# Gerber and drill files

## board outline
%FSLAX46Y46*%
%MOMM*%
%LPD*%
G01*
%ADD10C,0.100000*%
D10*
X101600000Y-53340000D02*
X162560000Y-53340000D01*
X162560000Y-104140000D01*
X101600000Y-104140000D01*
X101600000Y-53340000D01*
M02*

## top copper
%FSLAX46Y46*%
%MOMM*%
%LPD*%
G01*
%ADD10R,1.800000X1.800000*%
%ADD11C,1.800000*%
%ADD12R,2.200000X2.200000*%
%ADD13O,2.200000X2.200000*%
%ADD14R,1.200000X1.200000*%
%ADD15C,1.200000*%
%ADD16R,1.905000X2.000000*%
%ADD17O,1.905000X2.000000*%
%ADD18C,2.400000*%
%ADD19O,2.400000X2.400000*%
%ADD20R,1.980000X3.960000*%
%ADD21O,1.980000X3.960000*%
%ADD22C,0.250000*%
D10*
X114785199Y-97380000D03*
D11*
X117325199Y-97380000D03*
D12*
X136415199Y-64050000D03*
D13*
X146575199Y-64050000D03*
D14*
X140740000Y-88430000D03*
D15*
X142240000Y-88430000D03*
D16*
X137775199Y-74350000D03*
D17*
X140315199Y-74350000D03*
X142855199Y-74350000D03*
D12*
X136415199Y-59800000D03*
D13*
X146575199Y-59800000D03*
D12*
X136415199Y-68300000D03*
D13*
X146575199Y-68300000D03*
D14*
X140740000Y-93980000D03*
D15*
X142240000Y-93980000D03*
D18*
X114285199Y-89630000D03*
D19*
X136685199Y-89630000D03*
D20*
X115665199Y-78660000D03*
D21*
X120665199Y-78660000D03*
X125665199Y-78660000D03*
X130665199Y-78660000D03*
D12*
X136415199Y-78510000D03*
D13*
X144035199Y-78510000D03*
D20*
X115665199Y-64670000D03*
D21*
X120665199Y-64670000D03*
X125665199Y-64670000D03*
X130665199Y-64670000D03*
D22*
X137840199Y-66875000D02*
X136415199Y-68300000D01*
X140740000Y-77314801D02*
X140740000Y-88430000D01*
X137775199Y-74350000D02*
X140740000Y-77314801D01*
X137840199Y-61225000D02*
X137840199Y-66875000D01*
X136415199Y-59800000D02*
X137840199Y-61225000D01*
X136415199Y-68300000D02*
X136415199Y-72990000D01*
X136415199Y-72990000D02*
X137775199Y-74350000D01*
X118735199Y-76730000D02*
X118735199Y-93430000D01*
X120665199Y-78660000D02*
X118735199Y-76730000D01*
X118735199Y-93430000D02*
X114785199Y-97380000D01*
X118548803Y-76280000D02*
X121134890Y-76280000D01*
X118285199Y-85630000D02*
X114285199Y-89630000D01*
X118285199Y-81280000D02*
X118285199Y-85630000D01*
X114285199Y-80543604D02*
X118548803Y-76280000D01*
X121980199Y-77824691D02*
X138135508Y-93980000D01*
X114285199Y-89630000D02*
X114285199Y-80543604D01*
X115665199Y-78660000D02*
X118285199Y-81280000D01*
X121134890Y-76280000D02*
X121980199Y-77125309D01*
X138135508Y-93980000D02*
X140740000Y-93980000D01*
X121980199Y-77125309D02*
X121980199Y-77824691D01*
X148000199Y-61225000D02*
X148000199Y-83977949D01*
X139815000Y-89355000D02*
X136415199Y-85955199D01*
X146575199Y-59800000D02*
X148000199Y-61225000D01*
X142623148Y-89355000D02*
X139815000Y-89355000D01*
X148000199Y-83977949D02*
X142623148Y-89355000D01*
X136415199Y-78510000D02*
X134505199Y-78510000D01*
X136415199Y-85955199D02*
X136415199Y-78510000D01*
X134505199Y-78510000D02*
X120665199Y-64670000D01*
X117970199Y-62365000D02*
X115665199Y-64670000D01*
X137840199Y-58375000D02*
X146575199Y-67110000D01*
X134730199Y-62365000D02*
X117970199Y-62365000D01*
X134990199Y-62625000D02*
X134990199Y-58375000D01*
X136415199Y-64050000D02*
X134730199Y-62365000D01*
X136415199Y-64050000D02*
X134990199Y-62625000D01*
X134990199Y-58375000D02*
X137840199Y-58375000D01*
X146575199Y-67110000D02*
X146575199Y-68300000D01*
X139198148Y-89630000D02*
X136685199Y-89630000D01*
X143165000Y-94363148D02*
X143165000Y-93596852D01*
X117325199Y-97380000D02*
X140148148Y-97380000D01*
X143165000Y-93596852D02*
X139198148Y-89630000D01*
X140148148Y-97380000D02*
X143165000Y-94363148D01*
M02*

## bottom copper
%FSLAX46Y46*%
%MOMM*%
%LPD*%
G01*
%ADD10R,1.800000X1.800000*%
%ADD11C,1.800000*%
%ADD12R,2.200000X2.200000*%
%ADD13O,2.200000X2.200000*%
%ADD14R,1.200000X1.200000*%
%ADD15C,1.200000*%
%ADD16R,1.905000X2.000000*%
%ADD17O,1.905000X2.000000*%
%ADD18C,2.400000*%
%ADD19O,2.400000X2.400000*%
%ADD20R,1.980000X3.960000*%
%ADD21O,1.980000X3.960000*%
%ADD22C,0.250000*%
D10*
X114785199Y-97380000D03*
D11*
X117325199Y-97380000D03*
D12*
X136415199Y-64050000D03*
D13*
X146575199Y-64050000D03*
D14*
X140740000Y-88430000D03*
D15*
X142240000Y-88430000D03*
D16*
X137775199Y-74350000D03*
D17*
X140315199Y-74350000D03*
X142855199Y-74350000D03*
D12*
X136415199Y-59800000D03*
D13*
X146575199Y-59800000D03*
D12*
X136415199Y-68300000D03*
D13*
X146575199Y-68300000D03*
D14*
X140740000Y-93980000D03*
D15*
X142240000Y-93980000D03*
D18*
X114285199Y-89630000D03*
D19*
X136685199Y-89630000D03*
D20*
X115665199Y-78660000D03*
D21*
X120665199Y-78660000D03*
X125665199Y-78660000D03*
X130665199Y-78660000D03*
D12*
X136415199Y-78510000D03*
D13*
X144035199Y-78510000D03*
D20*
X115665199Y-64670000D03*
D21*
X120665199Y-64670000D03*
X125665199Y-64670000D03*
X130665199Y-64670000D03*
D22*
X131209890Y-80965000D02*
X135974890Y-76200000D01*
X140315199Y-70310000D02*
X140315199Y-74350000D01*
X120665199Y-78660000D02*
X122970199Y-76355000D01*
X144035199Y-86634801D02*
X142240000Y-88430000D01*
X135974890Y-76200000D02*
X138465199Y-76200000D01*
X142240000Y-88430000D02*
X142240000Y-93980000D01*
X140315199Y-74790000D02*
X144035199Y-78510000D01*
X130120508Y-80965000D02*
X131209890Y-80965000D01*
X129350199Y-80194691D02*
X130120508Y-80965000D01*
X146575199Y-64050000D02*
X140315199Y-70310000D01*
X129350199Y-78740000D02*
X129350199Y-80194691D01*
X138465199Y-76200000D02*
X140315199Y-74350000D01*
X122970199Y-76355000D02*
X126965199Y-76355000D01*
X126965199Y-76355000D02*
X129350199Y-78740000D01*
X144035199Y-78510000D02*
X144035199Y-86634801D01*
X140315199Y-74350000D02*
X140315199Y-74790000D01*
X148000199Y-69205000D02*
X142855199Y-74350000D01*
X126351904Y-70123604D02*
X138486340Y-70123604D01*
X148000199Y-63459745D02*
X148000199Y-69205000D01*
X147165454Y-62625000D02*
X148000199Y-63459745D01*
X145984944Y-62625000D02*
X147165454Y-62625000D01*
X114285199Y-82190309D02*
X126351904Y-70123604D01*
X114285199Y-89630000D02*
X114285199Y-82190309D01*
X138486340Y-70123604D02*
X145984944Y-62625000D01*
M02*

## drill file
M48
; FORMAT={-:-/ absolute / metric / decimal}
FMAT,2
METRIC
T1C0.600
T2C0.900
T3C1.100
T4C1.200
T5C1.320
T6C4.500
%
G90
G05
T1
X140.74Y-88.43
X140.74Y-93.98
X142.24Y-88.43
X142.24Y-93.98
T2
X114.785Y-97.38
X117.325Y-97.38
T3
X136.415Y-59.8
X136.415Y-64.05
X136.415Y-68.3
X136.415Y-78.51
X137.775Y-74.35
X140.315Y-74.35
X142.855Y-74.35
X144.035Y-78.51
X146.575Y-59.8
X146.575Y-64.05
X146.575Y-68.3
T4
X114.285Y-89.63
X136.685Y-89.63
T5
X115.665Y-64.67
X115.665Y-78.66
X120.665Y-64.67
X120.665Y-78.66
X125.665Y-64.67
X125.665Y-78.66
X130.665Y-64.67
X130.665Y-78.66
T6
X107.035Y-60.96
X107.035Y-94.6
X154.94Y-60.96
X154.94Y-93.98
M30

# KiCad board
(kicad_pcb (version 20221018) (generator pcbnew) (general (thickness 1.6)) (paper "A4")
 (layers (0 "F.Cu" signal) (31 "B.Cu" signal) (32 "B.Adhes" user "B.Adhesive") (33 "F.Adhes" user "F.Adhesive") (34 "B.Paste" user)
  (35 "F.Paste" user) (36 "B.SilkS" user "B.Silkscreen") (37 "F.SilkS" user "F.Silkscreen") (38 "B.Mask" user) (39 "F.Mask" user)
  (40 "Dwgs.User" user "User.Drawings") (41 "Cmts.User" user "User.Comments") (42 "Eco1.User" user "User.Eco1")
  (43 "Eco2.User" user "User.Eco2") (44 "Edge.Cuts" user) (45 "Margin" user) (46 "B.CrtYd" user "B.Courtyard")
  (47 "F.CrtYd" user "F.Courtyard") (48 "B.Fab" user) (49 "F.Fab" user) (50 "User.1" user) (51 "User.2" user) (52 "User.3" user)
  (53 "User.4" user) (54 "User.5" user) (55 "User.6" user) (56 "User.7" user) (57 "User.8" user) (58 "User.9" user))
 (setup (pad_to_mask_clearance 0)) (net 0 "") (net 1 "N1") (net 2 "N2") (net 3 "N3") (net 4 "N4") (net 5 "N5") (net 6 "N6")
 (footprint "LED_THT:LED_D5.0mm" (layer "F.Cu") (at 114.785199 97.38)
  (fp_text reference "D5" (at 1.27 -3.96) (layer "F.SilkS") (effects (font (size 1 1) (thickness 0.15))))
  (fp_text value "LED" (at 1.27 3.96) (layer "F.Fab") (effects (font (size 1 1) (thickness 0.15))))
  (pad "1" thru_hole rect (at 0 0) (size 1.8 1.8) (drill 0.9) (layers "*.Cu" "*.Mask") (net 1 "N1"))
  (pad "2" thru_hole circle (at 2.54 0) (size 1.8 1.8) (drill 0.9) (layers "*.Cu" "*.Mask") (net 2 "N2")))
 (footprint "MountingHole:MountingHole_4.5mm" (layer "F.Cu") (at 107.035199 60.96)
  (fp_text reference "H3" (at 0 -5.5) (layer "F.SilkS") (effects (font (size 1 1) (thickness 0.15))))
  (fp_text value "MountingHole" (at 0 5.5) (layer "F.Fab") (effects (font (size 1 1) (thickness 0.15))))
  (pad "" np_thru_hole circle (at 0 0) (size 4.5 4.5) (drill 4.5) (layers "*.Cu" "*.Mask")))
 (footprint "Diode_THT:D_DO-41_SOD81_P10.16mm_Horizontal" (layer "F.Cu") (at 136.415199 64.05)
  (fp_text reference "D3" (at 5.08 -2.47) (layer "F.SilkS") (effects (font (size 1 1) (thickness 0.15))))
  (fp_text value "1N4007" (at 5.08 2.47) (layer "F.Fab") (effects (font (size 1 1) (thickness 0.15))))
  (pad "1" thru_hole rect (at 0 0) (size 2.2 2.2) (drill 1.1) (layers "*.Cu" "*.Mask") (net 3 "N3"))
  (pad "2" thru_hole oval (at 10.16 0) (size 2.2 2.2) (drill 1.1) (layers "*.Cu" "*.Mask") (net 1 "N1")))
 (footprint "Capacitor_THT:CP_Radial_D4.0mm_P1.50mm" (layer "F.Cu") (at 140.74 88.43)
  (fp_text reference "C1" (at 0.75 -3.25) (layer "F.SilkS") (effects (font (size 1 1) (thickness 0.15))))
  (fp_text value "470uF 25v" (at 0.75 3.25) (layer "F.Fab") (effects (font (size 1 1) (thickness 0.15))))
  (pad "1" thru_hole rect (at 0 0) (size 1.2 1.2) (drill 0.6) (layers "*.Cu" "*.Mask") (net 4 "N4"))
  (pad "2" thru_hole circle (at 1.5 0) (size 1.2 1.2) (drill 0.6) (layers "*.Cu" "*.Mask") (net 1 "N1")))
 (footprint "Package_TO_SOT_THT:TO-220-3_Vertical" (layer "F.Cu") (at 137.775199 74.35)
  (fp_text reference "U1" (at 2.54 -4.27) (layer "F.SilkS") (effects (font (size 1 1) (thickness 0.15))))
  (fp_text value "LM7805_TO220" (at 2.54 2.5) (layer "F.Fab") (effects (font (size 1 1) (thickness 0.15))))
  (pad "1" thru_hole rect (at 0 0) (size 1.905 2) (drill 1.1) (layers "*.Cu" "*.Mask") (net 4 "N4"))
  (pad "2" thru_hole oval (at 2.54 0) (size 1.905 2) (drill 1.1) (layers "*.Cu" "*.Mask") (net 1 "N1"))
  (pad "3" thru_hole oval (at 5.08 0) (size 1.905 2) (drill 1.1) (layers "*.Cu" "*.Mask") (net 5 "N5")))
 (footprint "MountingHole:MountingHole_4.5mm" (layer "F.Cu") (at 154.94 93.98)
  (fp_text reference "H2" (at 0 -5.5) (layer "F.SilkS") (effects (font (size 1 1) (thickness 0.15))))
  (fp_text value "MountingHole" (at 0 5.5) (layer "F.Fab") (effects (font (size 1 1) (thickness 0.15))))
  (pad "" np_thru_hole circle (at 0 0) (size 4.5 4.5) (drill 4.5) (layers "*.Cu" "*.Mask")))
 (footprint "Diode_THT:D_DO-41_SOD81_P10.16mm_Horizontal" (layer "F.Cu") (at 136.415199 59.8)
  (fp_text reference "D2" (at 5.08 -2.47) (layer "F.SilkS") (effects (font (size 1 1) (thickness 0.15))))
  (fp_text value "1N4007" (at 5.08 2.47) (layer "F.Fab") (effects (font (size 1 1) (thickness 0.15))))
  (pad "1" thru_hole rect (at 0 0) (size 2.2 2.2) (drill 1.1) (layers "*.Cu" "*.Mask") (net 4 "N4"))
  (pad "2" thru_hole oval (at 10.16 0) (size 2.2 2.2) (drill 1.1) (layers "*.Cu" "*.Mask") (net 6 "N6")))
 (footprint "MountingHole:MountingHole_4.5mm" (layer "F.Cu") (at 154.94 60.96)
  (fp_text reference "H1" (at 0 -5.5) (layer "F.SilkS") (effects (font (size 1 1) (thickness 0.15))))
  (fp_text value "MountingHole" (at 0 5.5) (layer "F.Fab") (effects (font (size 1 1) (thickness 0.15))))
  (pad "" np_thru_hole circle (at 0 0) (size 4.5 4.5) (drill 4.5) (layers "*.Cu" "*.Mask")))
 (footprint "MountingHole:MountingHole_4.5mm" (layer "F.Cu") (at 107.035199 94.6)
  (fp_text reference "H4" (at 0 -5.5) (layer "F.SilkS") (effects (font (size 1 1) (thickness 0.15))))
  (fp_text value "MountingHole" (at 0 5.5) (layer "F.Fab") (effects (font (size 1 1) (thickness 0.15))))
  (pad "" np_thru_hole circle (at 0 0) (size 4.5 4.5) (drill 4.5) (layers "*.Cu" "*.Mask")))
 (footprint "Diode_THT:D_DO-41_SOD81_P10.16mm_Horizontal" (layer "F.Cu") (at 136.415199 68.3)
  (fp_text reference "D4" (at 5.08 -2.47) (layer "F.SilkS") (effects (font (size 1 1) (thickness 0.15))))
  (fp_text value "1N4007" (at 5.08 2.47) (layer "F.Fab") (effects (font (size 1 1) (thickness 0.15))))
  (pad "1" thru_hole rect (at 0 0) (size 2.2 2.2) (drill 1.1) (layers "*.Cu" "*.Mask") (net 4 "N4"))
  (pad "2" thru_hole oval (at 10.16 0) (size 2.2 2.2) (drill 1.1) (layers "*.Cu" "*.Mask") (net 3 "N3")))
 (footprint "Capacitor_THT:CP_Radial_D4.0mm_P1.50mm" (layer "F.Cu") (at 140.74 93.98)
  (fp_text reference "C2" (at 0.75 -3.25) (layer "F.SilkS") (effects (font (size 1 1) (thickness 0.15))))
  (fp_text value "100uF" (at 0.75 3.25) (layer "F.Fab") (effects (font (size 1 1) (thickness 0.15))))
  (pad "1" thru_hole rect (at 0 0) (size 1.2 1.2) (drill 0.6) (layers "*.Cu" "*.Mask") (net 5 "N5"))
  (pad "2" thru_hole circle (at 1.5 0) (size 1.2 1.2) (drill 0.6) (layers "*.Cu" "*.Mask") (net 1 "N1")))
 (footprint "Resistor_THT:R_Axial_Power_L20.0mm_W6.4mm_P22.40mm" (layer "F.Cu") (at 114.285199 89.63)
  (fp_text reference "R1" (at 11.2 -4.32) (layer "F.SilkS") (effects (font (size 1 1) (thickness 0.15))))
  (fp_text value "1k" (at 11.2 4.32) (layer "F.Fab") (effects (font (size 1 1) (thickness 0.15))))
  (pad "1" thru_hole circle (at 0 0) (size 2.4 2.4) (drill 1.2) (layers "*.Cu" "*.Mask") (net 5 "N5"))
  (pad "2" thru_hole oval (at 22.4 0) (size 2.4 2.4) (drill 1.2) (layers "*.Cu" "*.Mask") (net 2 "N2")))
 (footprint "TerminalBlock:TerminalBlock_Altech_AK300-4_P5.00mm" (layer "F.Cu") (at 115.665199 78.66)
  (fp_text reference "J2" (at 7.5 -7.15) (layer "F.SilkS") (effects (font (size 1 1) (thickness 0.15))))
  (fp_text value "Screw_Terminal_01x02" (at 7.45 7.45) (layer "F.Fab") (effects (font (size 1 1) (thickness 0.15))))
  (pad "1" thru_hole rect (at 0 0) (size 1.98 3.96) (drill 1.32) (layers "*.Cu" "*.Mask") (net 5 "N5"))
  (pad "2" thru_hole oval (at 5 0) (size 1.98 3.96) (drill 1.32) (layers "*.Cu" "*.Mask") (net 1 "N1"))
  (pad "3" thru_hole oval (at 10 0) (size 1.98 3.96) (drill 1.32) (layers "*.Cu" "*.Mask"))
  (pad "4" thru_hole oval (at 15 0) (size 1.98 3.96) (drill 1.32) (layers "*.Cu" "*.Mask")))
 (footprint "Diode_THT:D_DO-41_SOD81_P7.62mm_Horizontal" (layer "F.Cu") (at 136.415199 78.51)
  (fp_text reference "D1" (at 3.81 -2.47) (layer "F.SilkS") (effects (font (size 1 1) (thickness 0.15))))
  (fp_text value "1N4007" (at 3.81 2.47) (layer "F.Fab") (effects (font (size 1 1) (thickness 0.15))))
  (pad "1" thru_hole rect (at 0 0) (size 2.2 2.2) (drill 1.1) (layers "*.Cu" "*.Mask") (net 6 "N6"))
  (pad "2" thru_hole oval (at 7.62 0) (size 2.2 2.2) (drill 1.1) (layers "*.Cu" "*.Mask") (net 1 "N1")))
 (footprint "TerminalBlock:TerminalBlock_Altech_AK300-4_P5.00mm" (layer "F.Cu") (at 115.665199 64.67)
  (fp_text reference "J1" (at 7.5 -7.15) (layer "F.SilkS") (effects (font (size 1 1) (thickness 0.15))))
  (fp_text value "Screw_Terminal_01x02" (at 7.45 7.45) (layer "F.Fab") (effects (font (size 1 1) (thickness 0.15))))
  (pad "1" thru_hole rect (at 0 0) (size 1.98 3.96) (drill 1.32) (layers "*.Cu" "*.Mask") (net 3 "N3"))
  (pad "2" thru_hole oval (at 5 0) (size 1.98 3.96) (drill 1.32) (layers "*.Cu" "*.Mask") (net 6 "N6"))
  (pad "3" thru_hole oval (at 10 0) (size 1.98 3.96) (drill 1.32) (layers "*.Cu" "*.Mask"))
  (pad "4" thru_hole oval (at 15 0) (size 1.98 3.96) (drill 1.32) (layers "*.Cu" "*.Mask")))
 (gr_rect (start 101.6 53.34) (end 162.56 104.14) (stroke (width 0.1) (type default)) (fill none) (layer "Edge.Cuts"))
 (segment (start 137.840199 66.875) (end 136.415199 68.3) (width 0.25) (layer "F.Cu") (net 4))
 (segment (start 140.74 77.314801) (end 140.74 88.43) (width 0.25) (layer "F.Cu") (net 4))
 (segment (start 137.775199 74.35) (end 140.74 77.314801) (width 0.25) (layer "F.Cu") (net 4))
 (segment (start 137.840199 61.225) (end 137.840199 66.875) (width 0.25) (layer "F.Cu") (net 4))
 (segment (start 136.415199 59.8) (end 137.840199 61.225) (width 0.25) (layer "F.Cu") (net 4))
 (segment (start 136.415199 68.3) (end 136.415199 72.99) (width 0.25) (layer "F.Cu") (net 4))
 (segment (start 136.415199 72.99) (end 137.775199 74.35) (width 0.25) (layer "F.Cu") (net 4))
 (segment (start 118.735199 76.73) (end 118.735199 93.43) (width 0.25) (layer "F.Cu") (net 1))
 (segment (start 120.665199 78.66) (end 118.735199 76.73) (width 0.25) (layer "F.Cu") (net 1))
 (segment (start 118.735199 93.43) (end 114.785199 97.38) (width 0.25) (layer "F.Cu") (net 1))
 (segment (start 131.20989 80.965) (end 135.97489 76.2) (width 0.25) (layer "B.Cu") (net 1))
 (segment (start 140.315199 70.31) (end 140.315199 74.35) (width 0.25) (layer "B.Cu") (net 1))
 (segment (start 120.665199 78.66) (end 122.970199 76.355) (width 0.25) (layer "B.Cu") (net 1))
 (segment (start 144.035199 86.634801) (end 142.24 88.43) (width 0.25) (layer "B.Cu") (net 1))
 (segment (start 135.97489 76.2) (end 138.465199 76.2) (width 0.25) (layer "B.Cu") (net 1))
 (segment (start 142.24 88.43) (end 142.24 93.98) (width 0.25) (layer "B.Cu") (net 1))
 (segment (start 140.315199 74.79) (end 144.035199 78.51) (width 0.25) (layer "B.Cu") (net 1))
 (segment (start 130.120508 80.965) (end 131.20989 80.965) (width 0.25) (layer "B.Cu") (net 1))
 (segment (start 129.350199 80.194691) (end 130.120508 80.965) (width 0.25) (layer "B.Cu") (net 1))
 (segment (start 146.575199 64.05) (end 140.315199 70.31) (width 0.25) (layer "B.Cu") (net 1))
 (segment (start 129.350199 78.74) (end 129.350199 80.194691) (width 0.25) (layer "B.Cu") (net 1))
 (segment (start 138.465199 76.2) (end 140.315199 74.35) (width 0.25) (layer "B.Cu") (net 1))
 (segment (start 122.970199 76.355) (end 126.965199 76.355) (width 0.25) (layer "B.Cu") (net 1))
 (segment (start 126.965199 76.355) (end 129.350199 78.74) (width 0.25) (layer "B.Cu") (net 1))
 (segment (start 144.035199 78.51) (end 144.035199 86.634801) (width 0.25) (layer "B.Cu") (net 1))
 (segment (start 140.315199 74.35) (end 140.315199 74.79) (width 0.25) (layer "B.Cu") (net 1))
 (segment (start 118.548803 76.28) (end 121.13489 76.28) (width 0.25) (layer "F.Cu") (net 5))
 (segment (start 118.285199 85.63) (end 114.285199 89.63) (width 0.25) (layer "F.Cu") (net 5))
 (segment (start 118.285199 81.28) (end 118.285199 85.63) (width 0.25) (layer "F.Cu") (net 5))
 (segment (start 114.285199 80.543604) (end 118.548803 76.28) (width 0.25) (layer "F.Cu") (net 5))
 (segment (start 121.980199 77.824691) (end 138.135508 93.98) (width 0.25) (layer "F.Cu") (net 5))
 (segment (start 114.285199 89.63) (end 114.285199 80.543604) (width 0.25) (layer "F.Cu") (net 5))
 (segment (start 115.665199 78.66) (end 118.285199 81.28) (width 0.25) (layer "F.Cu") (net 5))
 (segment (start 121.13489 76.28) (end 121.980199 77.125309) (width 0.25) (layer "F.Cu") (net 5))
 (segment (start 138.135508 93.98) (end 140.74 93.98) (width 0.25) (layer "F.Cu") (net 5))
 (segment (start 121.980199 77.125309) (end 121.980199 77.824691) (width 0.25) (layer "F.Cu") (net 5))
 (segment (start 148.000199 69.205) (end 142.855199 74.35) (width 0.25) (layer "B.Cu") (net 5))
 (segment (start 126.351904 70.123604) (end 138.48634 70.123604) (width 0.25) (layer "B.Cu") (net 5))
 (segment (start 148.000199 63.459745) (end 148.000199 69.205) (width 0.25) (layer "B.Cu") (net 5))
 (segment (start 147.165454 62.625) (end 148.000199 63.459745) (width 0.25) (layer "B.Cu") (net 5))
 (segment (start 145.984944 62.625) (end 147.165454 62.625) (width 0.25) (layer "B.Cu") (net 5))
 (segment (start 114.285199 82.190309) (end 126.351904 70.123604) (width 0.25) (layer "B.Cu") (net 5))
 (segment (start 114.285199 89.63) (end 114.285199 82.190309) (width 0.25) (layer "B.Cu") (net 5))
 (segment (start 138.48634 70.123604) (end 145.984944 62.625) (width 0.25) (layer "B.Cu") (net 5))
 (segment (start 148.000199 61.225) (end 148.000199 83.977949) (width 0.25) (layer "F.Cu") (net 6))
 (segment (start 139.815 89.355) (end 136.415199 85.955199) (width 0.25) (layer "F.Cu") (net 6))
 (segment (start 146.575199 59.8) (end 148.000199 61.225) (width 0.25) (layer "F.Cu") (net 6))
 (segment (start 142.623148 89.355) (end 139.815 89.355) (width 0.25) (layer "F.Cu") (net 6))
 (segment (start 148.000199 83.977949) (end 142.623148 89.355) (width 0.25) (layer "F.Cu") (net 6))
 (segment (start 136.415199 78.51) (end 134.505199 78.51) (width 0.25) (layer "F.Cu") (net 6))
 (segment (start 136.415199 85.955199) (end 136.415199 78.51) (width 0.25) (layer "F.Cu") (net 6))
 (segment (start 134.505199 78.51) (end 120.665199 64.67) (width 0.25) (layer "F.Cu") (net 6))
 (segment (start 117.970199 62.365) (end 115.665199 64.67) (width 0.25) (layer "F.Cu") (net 3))
 (segment (start 137.840199 58.375) (end 146.575199 67.11) (width 0.25) (layer "F.Cu") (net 3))
 (segment (start 134.730199 62.365) (end 117.970199 62.365) (width 0.25) (layer "F.Cu") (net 3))
 (segment (start 134.990199 62.625) (end 134.990199 58.375) (width 0.25) (layer "F.Cu") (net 3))
 (segment (start 136.415199 64.05) (end 134.730199 62.365) (width 0.25) (layer "F.Cu") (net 3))
 (segment (start 136.415199 64.05) (end 134.990199 62.625) (width 0.25) (layer "F.Cu") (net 3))
 (segment (start 134.990199 58.375) (end 137.840199 58.375) (width 0.25) (layer "F.Cu") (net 3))
 (segment (start 146.575199 67.11) (end 146.575199 68.3) (width 0.25) (layer "F.Cu") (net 3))
 (segment (start 139.198148 89.63) (end 136.685199 89.63) (width 0.25) (layer "F.Cu") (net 2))
 (segment (start 143.165 94.363148) (end 143.165 93.596852) (width 0.25) (layer "F.Cu") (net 2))
 (segment (start 117.325199 97.38) (end 140.148148 97.38) (width 0.25) (layer "F.Cu") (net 2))
 (segment (start 143.165 93.596852) (end 139.198148 89.63) (width 0.25) (layer "F.Cu") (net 2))
 (segment (start 140.148148 97.38) (end 143.165 94.363148) (width 0.25) (layer "F.Cu") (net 2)))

